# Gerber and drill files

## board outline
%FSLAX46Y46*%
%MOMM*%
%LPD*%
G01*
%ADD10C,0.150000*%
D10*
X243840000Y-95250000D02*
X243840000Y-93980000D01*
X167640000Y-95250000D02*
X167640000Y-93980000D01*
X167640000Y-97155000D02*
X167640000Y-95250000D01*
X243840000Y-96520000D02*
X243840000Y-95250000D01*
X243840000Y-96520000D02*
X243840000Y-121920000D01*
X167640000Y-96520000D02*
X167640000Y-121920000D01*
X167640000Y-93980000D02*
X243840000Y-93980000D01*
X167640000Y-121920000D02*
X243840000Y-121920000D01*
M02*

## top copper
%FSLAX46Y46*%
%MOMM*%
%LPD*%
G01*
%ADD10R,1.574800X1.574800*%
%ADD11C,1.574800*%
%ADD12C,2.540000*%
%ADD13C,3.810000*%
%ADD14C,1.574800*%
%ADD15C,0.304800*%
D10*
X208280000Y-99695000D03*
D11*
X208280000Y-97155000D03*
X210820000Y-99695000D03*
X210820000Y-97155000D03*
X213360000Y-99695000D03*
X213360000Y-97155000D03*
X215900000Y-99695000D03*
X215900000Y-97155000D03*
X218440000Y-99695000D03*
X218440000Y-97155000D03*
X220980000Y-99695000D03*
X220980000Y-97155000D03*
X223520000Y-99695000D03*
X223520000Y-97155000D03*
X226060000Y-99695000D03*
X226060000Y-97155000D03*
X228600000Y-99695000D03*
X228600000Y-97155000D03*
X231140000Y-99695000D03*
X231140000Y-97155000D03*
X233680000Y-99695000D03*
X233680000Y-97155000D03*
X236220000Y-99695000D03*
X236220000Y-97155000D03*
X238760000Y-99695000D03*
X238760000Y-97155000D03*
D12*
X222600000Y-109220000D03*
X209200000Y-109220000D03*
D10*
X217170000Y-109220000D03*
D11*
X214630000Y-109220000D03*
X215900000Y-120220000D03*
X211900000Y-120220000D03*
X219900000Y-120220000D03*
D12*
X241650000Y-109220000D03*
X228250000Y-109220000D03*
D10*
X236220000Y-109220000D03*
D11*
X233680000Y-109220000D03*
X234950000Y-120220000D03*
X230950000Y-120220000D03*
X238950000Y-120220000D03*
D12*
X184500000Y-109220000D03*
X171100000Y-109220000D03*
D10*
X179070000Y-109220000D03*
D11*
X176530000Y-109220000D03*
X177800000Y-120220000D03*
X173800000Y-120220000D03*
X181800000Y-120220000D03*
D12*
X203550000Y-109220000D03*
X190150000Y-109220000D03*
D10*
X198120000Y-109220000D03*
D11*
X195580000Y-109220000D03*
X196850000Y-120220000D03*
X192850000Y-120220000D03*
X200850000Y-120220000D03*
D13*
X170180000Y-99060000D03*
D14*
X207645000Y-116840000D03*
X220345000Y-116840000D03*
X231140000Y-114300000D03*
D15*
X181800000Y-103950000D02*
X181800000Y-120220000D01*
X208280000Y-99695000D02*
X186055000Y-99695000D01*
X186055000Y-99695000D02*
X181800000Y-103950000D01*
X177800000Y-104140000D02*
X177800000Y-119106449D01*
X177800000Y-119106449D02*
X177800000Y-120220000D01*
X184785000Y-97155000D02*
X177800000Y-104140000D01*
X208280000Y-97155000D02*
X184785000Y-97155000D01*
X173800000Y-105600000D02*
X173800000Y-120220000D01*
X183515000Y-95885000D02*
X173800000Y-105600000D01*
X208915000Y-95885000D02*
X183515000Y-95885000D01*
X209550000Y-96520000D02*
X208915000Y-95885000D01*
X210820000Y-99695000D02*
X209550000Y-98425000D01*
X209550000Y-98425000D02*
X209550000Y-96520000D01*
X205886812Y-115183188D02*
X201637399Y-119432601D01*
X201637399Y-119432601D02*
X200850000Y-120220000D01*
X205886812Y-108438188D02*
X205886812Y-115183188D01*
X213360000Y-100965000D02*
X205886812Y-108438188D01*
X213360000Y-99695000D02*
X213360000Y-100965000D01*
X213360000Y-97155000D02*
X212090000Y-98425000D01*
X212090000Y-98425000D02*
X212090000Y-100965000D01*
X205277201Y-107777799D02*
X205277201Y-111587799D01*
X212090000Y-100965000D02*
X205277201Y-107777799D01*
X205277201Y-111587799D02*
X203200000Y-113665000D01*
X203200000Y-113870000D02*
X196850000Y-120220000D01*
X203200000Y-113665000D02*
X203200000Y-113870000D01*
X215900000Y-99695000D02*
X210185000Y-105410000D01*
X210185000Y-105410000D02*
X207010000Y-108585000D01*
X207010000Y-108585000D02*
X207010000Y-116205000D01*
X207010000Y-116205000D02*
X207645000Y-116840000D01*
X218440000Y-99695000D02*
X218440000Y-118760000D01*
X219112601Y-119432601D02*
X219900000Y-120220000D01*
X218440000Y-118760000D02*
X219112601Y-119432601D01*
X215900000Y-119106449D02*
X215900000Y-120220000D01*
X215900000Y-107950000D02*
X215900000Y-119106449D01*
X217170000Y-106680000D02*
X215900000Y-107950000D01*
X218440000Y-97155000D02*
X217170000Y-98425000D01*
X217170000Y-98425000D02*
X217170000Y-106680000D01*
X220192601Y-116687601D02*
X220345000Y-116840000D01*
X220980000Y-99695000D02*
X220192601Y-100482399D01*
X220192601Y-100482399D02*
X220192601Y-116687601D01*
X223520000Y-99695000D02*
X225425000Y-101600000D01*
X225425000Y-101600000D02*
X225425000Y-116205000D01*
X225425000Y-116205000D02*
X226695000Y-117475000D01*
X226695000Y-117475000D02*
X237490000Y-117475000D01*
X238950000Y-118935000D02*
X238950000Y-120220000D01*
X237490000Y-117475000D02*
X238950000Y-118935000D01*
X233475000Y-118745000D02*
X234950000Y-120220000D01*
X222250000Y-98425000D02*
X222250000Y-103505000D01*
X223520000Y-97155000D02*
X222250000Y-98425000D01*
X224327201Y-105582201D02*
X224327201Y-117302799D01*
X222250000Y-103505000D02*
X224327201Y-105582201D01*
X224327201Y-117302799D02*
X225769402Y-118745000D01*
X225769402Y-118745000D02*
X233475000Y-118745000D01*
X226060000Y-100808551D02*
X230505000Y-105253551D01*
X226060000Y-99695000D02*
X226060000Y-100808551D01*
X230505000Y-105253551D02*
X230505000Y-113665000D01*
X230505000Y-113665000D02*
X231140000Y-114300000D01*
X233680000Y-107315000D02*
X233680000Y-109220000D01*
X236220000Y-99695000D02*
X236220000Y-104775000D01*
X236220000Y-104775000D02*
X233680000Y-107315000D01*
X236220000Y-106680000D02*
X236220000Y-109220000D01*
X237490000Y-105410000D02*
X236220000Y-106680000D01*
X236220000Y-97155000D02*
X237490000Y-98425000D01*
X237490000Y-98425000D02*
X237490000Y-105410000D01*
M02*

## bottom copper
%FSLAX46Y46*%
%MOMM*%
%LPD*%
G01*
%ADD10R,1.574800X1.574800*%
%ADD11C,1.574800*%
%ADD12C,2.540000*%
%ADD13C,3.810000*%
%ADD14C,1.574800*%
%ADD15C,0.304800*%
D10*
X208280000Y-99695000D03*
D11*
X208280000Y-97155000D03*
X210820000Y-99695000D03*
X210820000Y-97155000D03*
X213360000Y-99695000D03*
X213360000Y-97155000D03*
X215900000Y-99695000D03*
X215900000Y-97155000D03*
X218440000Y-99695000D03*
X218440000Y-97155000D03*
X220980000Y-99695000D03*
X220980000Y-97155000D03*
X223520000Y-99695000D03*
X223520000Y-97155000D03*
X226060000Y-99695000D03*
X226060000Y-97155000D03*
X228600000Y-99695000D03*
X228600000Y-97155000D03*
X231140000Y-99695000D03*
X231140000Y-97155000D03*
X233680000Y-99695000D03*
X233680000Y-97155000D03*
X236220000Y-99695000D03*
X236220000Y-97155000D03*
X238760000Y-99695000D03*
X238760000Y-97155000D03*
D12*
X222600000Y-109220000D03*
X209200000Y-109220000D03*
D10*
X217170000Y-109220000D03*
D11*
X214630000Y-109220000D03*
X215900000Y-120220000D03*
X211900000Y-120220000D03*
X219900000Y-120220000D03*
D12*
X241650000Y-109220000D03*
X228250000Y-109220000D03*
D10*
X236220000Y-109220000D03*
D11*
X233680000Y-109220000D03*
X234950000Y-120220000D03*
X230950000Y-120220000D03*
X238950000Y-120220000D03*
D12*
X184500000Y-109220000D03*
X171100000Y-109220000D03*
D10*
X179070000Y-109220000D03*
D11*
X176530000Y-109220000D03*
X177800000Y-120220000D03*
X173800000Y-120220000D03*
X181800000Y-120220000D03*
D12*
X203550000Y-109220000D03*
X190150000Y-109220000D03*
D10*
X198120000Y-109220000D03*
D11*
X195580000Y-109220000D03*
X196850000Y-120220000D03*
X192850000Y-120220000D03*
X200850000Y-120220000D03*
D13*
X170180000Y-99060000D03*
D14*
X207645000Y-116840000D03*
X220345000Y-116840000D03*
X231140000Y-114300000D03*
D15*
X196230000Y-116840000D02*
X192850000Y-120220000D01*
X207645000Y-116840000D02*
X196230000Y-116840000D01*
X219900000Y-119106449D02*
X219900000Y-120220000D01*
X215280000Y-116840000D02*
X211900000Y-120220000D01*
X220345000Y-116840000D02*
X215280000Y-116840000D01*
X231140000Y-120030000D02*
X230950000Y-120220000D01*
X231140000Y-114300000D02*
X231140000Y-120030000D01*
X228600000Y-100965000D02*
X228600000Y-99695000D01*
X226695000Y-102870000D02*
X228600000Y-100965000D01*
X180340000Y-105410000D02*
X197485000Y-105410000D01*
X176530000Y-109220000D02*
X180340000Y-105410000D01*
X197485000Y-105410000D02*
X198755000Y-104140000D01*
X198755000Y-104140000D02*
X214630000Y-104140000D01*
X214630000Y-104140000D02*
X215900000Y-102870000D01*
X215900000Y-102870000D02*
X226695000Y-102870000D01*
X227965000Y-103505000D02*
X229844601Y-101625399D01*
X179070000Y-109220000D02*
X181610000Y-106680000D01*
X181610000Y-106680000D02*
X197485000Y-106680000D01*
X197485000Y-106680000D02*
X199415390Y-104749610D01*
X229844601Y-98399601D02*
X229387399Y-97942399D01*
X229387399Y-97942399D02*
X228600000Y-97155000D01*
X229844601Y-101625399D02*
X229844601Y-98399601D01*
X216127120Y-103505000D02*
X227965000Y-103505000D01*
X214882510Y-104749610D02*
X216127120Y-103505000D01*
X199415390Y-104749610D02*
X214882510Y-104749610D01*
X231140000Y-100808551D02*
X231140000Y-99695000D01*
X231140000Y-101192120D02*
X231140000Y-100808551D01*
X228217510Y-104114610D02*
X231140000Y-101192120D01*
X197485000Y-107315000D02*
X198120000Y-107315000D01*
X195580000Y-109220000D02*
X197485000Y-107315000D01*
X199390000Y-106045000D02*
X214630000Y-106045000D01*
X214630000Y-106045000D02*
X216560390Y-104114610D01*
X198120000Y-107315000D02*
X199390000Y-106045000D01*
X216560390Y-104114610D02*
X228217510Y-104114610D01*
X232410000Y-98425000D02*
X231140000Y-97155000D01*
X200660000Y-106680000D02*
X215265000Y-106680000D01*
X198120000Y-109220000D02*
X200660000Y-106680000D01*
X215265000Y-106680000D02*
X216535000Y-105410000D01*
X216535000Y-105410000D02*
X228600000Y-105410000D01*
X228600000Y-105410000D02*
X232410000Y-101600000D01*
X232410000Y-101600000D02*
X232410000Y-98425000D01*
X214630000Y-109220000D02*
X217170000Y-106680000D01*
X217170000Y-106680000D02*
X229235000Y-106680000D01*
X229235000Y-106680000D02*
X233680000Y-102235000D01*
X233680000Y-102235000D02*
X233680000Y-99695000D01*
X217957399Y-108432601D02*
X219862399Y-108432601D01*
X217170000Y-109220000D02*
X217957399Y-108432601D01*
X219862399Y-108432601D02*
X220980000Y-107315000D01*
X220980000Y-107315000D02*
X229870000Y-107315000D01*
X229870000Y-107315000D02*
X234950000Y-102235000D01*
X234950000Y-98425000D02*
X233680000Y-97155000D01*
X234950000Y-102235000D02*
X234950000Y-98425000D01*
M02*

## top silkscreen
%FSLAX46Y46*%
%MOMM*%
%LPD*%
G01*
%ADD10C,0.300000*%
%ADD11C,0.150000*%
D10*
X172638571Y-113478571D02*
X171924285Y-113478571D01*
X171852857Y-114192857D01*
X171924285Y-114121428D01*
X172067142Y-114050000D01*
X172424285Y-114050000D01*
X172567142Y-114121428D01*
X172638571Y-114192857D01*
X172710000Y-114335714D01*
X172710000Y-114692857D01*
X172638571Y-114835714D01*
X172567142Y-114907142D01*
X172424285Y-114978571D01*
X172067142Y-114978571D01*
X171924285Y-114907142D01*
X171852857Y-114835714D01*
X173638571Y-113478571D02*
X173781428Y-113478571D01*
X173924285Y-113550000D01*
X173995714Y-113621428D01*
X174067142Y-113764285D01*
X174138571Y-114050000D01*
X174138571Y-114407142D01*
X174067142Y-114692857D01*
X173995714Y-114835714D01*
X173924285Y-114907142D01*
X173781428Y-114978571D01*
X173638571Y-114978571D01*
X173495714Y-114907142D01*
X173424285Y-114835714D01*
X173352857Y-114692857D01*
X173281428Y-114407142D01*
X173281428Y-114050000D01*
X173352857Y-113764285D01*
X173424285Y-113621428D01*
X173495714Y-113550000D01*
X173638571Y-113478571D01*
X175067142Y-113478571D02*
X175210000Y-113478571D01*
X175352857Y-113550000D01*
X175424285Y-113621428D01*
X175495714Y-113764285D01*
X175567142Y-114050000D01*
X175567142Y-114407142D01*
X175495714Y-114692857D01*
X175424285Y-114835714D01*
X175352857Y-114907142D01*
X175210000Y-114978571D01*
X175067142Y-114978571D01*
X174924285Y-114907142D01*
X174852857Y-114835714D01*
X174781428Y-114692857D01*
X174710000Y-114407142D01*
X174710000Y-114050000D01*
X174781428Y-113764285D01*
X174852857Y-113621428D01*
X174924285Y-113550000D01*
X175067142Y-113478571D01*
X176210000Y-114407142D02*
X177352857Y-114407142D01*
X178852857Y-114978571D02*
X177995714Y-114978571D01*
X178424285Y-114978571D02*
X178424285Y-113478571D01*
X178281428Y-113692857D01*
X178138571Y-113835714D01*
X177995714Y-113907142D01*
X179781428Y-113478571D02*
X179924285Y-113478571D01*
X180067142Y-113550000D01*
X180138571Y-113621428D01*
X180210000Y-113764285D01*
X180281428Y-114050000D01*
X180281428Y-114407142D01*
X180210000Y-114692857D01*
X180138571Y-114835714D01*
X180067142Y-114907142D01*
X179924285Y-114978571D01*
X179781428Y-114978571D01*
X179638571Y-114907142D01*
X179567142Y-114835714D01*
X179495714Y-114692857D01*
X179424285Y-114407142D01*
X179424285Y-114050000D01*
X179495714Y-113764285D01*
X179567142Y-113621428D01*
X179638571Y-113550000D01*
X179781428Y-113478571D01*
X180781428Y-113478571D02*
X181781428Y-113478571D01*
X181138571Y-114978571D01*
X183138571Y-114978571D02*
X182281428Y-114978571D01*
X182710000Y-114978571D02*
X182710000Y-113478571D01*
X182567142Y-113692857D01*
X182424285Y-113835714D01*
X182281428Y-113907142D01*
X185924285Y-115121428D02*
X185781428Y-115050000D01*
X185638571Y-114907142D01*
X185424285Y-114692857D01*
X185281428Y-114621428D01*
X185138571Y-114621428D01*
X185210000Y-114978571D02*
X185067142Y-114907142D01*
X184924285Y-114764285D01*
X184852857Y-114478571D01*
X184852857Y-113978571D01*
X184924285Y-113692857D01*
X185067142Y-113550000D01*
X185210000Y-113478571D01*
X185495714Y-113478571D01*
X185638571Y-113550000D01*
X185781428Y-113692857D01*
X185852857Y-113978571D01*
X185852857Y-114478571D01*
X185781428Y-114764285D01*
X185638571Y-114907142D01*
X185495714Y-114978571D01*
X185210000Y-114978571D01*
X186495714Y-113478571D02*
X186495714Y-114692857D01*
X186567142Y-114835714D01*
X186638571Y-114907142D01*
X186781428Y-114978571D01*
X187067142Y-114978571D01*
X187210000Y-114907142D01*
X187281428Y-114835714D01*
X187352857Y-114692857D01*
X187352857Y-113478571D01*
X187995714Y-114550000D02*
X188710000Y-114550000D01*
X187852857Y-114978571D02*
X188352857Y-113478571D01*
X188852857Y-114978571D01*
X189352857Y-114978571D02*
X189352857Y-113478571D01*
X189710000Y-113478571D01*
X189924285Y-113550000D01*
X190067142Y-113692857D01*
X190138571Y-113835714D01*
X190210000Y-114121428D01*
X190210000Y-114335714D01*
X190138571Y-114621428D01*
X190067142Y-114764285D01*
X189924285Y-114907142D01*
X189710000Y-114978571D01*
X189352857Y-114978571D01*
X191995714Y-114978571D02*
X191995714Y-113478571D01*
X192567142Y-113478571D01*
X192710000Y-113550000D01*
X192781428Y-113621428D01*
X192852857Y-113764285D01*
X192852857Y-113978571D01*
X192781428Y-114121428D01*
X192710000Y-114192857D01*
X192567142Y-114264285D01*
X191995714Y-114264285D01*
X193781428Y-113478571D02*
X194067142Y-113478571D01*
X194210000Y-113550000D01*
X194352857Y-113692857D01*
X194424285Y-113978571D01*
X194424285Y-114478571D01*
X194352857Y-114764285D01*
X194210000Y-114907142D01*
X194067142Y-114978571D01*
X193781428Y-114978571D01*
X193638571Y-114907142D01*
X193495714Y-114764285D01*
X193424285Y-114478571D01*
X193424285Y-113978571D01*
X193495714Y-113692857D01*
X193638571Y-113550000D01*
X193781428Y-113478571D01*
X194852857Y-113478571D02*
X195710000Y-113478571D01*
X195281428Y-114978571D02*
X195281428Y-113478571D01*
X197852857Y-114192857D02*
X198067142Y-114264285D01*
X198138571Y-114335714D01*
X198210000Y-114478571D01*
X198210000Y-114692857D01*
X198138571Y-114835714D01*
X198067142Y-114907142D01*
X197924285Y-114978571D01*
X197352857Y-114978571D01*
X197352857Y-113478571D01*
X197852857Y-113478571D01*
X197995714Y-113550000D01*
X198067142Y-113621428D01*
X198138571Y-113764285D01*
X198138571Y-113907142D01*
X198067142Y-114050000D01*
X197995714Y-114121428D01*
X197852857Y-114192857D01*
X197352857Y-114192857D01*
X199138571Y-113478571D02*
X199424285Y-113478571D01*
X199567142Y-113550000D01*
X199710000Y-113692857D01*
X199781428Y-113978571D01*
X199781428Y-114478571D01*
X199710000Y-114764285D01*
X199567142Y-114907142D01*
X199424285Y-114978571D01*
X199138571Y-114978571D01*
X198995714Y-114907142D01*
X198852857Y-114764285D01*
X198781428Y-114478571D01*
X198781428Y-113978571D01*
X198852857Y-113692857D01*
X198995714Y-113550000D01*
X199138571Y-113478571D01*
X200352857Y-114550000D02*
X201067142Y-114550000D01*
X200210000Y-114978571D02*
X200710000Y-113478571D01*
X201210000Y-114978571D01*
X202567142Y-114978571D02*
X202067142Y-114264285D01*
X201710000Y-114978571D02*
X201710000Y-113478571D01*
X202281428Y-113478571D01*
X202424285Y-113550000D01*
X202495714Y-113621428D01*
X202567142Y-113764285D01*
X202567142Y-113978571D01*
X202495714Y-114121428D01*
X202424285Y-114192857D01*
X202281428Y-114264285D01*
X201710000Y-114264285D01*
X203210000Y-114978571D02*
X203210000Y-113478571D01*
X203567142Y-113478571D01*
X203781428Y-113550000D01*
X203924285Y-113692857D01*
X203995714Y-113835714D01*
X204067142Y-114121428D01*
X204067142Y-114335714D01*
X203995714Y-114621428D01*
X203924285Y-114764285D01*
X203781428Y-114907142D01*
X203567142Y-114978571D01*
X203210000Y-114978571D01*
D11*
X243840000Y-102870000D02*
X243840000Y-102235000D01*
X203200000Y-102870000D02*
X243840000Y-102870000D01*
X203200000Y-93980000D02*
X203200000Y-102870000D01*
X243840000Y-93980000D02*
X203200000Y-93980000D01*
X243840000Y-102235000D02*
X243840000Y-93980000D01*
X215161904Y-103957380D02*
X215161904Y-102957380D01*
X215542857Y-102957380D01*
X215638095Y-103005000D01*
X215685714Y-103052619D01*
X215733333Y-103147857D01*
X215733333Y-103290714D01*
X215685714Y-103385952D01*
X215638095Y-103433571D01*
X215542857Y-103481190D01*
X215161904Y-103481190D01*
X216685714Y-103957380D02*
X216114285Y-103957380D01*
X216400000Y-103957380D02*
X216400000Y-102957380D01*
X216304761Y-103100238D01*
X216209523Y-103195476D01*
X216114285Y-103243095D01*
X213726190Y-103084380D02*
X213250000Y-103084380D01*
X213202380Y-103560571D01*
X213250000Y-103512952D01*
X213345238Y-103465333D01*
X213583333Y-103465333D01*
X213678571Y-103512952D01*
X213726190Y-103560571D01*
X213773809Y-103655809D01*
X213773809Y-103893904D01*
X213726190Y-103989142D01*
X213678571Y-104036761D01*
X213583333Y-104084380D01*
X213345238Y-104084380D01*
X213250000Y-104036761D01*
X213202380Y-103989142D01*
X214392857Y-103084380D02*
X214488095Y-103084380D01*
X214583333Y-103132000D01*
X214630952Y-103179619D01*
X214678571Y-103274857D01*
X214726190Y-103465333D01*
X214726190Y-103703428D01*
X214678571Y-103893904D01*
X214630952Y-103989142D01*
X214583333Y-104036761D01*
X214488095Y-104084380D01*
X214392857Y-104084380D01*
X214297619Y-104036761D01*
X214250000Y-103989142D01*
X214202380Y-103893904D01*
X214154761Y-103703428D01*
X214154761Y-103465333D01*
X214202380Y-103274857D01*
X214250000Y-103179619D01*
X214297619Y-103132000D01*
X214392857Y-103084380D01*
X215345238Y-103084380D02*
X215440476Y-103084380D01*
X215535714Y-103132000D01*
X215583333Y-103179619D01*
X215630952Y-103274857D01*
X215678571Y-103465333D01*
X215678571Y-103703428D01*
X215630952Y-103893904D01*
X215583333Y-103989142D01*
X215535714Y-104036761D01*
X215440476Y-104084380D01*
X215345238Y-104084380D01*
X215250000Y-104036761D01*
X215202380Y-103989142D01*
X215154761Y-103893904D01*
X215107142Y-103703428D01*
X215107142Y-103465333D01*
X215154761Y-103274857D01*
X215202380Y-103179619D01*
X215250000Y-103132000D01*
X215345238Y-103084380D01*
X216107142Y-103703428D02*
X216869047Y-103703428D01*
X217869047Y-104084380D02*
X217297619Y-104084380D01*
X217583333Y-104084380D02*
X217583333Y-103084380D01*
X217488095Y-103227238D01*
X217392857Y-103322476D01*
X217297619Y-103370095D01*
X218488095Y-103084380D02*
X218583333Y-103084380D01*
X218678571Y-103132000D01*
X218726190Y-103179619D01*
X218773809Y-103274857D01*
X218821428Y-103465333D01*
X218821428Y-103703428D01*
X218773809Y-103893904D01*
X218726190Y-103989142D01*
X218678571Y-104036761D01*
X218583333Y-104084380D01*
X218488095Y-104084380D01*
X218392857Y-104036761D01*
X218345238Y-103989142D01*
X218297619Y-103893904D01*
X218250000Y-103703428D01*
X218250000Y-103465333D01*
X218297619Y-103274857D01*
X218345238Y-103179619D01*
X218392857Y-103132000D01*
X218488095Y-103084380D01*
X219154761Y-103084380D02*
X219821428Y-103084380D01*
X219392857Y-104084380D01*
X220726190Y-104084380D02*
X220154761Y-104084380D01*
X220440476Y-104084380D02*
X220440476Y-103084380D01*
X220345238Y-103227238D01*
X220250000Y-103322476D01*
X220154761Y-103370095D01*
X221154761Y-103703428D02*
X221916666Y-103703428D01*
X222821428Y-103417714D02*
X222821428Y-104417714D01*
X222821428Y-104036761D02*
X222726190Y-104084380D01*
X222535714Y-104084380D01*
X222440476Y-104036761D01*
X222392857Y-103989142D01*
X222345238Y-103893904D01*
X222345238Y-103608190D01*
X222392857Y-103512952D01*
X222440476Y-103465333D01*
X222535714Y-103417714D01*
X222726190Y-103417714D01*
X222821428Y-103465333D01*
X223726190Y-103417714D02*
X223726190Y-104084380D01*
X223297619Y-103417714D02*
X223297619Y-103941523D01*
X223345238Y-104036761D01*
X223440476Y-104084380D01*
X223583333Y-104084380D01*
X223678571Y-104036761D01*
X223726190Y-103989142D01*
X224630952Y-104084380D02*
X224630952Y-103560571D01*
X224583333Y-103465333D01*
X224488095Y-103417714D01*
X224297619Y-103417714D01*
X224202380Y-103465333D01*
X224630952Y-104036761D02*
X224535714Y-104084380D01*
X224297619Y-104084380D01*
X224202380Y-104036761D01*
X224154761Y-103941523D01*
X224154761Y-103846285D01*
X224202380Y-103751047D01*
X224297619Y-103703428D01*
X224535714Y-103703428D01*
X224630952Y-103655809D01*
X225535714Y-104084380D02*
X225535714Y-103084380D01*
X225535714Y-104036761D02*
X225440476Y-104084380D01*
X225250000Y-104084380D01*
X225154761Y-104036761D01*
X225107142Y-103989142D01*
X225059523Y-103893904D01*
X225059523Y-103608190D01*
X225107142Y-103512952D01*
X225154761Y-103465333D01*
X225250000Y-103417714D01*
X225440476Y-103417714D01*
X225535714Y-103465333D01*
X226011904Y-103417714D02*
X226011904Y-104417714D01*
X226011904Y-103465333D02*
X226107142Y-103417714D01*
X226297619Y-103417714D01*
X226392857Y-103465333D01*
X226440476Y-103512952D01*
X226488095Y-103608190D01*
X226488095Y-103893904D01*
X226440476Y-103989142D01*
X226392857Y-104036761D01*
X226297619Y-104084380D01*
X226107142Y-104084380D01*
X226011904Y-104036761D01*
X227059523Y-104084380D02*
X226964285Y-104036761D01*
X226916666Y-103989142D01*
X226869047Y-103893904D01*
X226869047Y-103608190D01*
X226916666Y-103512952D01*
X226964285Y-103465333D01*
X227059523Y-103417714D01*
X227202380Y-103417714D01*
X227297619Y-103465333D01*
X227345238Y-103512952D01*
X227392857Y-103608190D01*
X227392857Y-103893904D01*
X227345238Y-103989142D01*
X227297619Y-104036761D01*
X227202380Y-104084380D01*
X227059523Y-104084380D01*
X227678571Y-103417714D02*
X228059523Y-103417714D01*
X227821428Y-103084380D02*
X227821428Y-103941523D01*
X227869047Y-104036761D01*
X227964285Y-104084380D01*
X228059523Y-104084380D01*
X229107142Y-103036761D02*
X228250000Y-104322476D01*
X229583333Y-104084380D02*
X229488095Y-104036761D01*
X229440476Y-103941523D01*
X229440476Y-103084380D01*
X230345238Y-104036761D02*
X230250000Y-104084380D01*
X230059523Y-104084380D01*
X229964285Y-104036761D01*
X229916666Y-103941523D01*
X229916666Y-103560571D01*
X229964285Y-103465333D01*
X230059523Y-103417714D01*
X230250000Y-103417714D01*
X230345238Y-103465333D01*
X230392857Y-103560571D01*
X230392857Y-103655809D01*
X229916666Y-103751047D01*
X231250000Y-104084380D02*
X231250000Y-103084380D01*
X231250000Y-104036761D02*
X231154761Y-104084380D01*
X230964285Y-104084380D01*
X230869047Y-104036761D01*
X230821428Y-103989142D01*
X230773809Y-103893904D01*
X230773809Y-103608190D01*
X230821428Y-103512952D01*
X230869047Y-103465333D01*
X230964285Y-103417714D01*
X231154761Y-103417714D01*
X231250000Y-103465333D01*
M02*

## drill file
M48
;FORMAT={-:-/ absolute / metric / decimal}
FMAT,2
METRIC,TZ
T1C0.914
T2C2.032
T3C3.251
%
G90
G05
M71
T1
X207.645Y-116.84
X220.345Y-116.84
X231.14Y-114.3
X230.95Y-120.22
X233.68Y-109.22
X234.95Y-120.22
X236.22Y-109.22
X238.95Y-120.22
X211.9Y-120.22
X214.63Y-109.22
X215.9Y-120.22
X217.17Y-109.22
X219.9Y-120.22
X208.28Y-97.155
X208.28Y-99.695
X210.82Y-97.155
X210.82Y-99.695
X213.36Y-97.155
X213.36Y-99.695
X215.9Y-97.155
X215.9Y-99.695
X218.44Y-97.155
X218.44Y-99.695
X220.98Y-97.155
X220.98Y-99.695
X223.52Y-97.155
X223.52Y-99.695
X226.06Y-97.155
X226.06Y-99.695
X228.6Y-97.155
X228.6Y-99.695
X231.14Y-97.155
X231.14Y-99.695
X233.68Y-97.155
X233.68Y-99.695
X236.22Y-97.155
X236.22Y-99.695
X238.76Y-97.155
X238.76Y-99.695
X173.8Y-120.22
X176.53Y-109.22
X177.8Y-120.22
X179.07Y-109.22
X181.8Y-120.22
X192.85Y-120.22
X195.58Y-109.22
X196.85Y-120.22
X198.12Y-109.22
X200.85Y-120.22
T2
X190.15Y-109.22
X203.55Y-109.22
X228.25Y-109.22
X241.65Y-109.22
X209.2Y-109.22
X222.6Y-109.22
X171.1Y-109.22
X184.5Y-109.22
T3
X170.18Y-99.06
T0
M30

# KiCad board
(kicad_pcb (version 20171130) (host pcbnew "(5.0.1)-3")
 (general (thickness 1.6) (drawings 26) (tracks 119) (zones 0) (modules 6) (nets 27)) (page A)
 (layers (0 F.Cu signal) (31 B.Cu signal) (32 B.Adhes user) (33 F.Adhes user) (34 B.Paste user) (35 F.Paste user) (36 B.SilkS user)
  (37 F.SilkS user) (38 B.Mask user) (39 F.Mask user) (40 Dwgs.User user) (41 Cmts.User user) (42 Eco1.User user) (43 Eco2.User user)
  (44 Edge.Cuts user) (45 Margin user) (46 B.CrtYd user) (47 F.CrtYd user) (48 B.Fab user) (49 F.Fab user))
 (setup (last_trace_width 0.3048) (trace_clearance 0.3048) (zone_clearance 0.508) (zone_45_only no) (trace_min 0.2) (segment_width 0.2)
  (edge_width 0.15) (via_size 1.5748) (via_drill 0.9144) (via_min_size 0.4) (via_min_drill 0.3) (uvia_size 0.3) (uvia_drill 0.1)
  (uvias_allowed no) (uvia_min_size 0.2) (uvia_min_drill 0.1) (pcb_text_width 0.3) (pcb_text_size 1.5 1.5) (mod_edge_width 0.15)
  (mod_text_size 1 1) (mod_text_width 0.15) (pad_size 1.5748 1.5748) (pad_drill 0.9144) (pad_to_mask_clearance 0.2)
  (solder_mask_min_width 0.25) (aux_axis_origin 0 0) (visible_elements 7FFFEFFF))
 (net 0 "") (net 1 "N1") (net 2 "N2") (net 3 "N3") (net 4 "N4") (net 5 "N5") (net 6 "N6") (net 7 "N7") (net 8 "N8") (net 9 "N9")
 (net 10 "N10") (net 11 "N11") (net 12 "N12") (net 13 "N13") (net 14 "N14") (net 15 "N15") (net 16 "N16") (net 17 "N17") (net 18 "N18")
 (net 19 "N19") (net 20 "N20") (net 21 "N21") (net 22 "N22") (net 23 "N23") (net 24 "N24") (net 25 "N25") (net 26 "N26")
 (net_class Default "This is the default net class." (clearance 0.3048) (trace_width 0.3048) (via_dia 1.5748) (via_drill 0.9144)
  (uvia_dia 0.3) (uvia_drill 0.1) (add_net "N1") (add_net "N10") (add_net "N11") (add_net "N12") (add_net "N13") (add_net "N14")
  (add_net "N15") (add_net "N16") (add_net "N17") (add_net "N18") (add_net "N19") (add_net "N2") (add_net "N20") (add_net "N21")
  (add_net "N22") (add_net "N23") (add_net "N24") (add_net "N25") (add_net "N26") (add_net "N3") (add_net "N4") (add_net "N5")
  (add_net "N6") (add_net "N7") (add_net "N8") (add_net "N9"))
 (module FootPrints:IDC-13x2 (layer F.Cu) (at 215.9 99.695)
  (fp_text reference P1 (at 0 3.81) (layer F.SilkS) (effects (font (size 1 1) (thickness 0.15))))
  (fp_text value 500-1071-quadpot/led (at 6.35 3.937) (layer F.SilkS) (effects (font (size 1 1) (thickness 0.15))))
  (fp_line (start 27.94 3.175) (end 27.94 2.54) (layer F.SilkS) (width 0.15))
  (fp_line (start -12.7 3.175) (end 27.94 3.175) (layer F.SilkS) (width 0.15))
  (fp_line (start -12.7 -5.715) (end -12.7 3.175) (layer F.SilkS) (width 0.15))
  (fp_line (start 27.94 -5.715) (end -12.7 -5.715) (layer F.SilkS) (width 0.15))
  (fp_line (start 27.94 2.54) (end 27.94 -5.715) (layer F.SilkS) (width 0.15))
  (pad 1 thru_hole rect (at -7.62 0) (size 1.5748 1.5748) (drill 0.9144) (layers *.Cu *.Mask) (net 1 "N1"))
  (pad 2 thru_hole circle (at -7.62 -2.54) (size 1.5748 1.5748) (drill 0.9144) (layers *.Cu *.Mask) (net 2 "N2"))
  (pad 3 thru_hole circle (at -5.08 0) (size 1.5748 1.5748) (drill 0.9144) (layers *.Cu *.Mask) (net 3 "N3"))
  (pad 4 thru_hole circle (at -5.08 -2.54) (size 1.5748 1.5748) (drill 0.9144) (layers *.Cu *.Mask) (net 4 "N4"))
  (pad 5 thru_hole circle (at -2.54 0) (size 1.5748 1.5748) (drill 0.9144) (layers *.Cu *.Mask) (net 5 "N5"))
  (pad 6 thru_hole circle (at -2.54 -2.54) (size 1.5748 1.5748) (drill 0.9144) (layers *.Cu *.Mask) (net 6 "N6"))
  (pad 7 thru_hole circle (at 0 0) (size 1.5748 1.5748) (drill 0.9144) (layers *.Cu *.Mask) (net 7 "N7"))
  (pad 8 thru_hole circle (at 0 -2.54) (size 1.5748 1.5748) (drill 0.9144) (layers *.Cu *.Mask) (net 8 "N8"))
  (pad 9 thru_hole circle (at 2.54 0) (size 1.5748 1.5748) (drill 0.9144) (layers *.Cu *.Mask) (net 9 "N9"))
  (pad 10 thru_hole circle (at 2.54 -2.54) (size 1.5748 1.5748) (drill 0.9144) (layers *.Cu *.Mask) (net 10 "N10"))
  (pad 11 thru_hole circle (at 5.08 0) (size 1.5748 1.5748) (drill 0.9144) (layers *.Cu *.Mask) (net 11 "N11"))
  (pad 12 thru_hole circle (at 5.08 -2.54) (size 1.5748 1.5748) (drill 0.9144) (layers *.Cu *.Mask) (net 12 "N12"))
  (pad 13 thru_hole circle (at 7.62 0) (size 1.5748 1.5748) (drill 0.9144) (layers *.Cu *.Mask) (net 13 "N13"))
  (pad 14 thru_hole circle (at 7.62 -2.54) (size 1.5748 1.5748) (drill 0.9144) (layers *.Cu *.Mask) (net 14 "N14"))
  (pad 15 thru_hole circle (at 10.16 0) (size 1.5748 1.5748) (drill 0.9144) (layers *.Cu *.Mask) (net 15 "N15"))
  (pad 16 thru_hole circle (at 10.16 -2.54) (size 1.5748 1.5748) (drill 0.9144) (layers *.Cu *.Mask) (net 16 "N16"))
  (pad 17 thru_hole circle (at 12.7 0) (size 1.5748 1.5748) (drill 0.9144) (layers *.Cu *.Mask) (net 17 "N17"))
  (pad 18 thru_hole circle (at 12.7 -2.54) (size 1.5748 1.5748) (drill 0.9144) (layers *.Cu *.Mask) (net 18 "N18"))
  (pad 19 thru_hole circle (at 15.24 0) (size 1.5748 1.5748) (drill 0.9144) (layers *.Cu *.Mask) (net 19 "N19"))
  (pad 20 thru_hole circle (at 15.24 -2.54) (size 1.5748 1.5748) (drill 0.9144) (layers *.Cu *.Mask) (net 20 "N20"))
  (pad 21 thru_hole circle (at 17.78 0) (size 1.5748 1.5748) (drill 0.9144) (layers *.Cu *.Mask) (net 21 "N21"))
  (pad 22 thru_hole circle (at 17.78 -2.54) (size 1.5748 1.5748) (drill 0.9144) (layers *.Cu *.Mask) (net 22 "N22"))
  (pad 23 thru_hole circle (at 20.32 0) (size 1.5748 1.5748) (drill 0.9144) (layers *.Cu *.Mask) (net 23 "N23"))
  (pad 24 thru_hole circle (at 20.32 -2.54) (size 1.5748 1.5748) (drill 0.9144) (layers *.Cu *.Mask) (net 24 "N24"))
  (pad 25 thru_hole circle (at 22.86 0) (size 1.5748 1.5748) (drill 0.9144) (layers *.Cu *.Mask) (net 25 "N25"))
  (pad 26 thru_hole circle (at 22.86 -2.54) (size 1.5748 1.5748) (drill 0.9144) (layers *.Cu *.Mask) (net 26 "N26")))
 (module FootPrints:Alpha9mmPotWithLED (layer B.Cu) (at 215.9 109.22 180)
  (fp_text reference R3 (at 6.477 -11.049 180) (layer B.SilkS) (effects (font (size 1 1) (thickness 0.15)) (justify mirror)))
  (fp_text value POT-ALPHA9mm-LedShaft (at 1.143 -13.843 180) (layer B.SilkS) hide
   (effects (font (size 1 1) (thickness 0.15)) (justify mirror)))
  (pad "" thru_hole circle (at -6.7 0 180) (size 2.54 2.54) (drill 2.032) (layers *.Cu *.Mask B.SilkS))
  (pad "" thru_hole circle (at 6.7 0 180) (size 2.54 2.54) (drill 2.032) (layers *.Cu *.Mask B.SilkS))
  (pad 4 thru_hole rect (at -1.27 0 180) (size 1.5748 1.5748) (drill 0.9144) (layers *.Cu *.Mask B.SilkS) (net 22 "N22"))
  (pad 5 thru_hole circle (at 1.27 0 180) (size 1.5748 1.5748) (drill 0.9144) (layers *.Cu *.Mask B.SilkS) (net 21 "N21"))
  (pad 2 thru_hole circle (at 0 -11 180) (size 1.5748 1.5748) (drill 0.9144) (layers *.Cu *.Mask B.SilkS) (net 10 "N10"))
  (pad 3 thru_hole circle (at 4 -11 180) (size 1.5748 1.5748) (drill 0.9144) (layers *.Cu *.Mask B.SilkS) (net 11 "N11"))
  (pad 1 thru_hole circle (at -4 -11 180) (size 1.5748 1.5748) (drill 0.9144) (layers *.Cu *.Mask B.SilkS) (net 9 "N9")))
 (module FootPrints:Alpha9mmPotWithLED (layer B.Cu) (at 234.95 109.22 180)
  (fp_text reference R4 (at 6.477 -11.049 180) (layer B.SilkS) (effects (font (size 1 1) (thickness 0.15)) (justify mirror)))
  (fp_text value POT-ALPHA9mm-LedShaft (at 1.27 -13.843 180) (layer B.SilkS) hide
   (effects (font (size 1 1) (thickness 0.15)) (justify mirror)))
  (pad "" thru_hole circle (at -6.7 0 180) (size 2.54 2.54) (drill 2.032) (layers *.Cu *.Mask B.SilkS))
  (pad "" thru_hole circle (at 6.7 0 180) (size 2.54 2.54) (drill 2.032) (layers *.Cu *.Mask B.SilkS))
  (pad 4 thru_hole rect (at -1.27 0 180) (size 1.5748 1.5748) (drill 0.9144) (layers *.Cu *.Mask B.SilkS) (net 24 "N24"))
  (pad 5 thru_hole circle (at 1.27 0 180) (size 1.5748 1.5748) (drill 0.9144) (layers *.Cu *.Mask B.SilkS) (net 23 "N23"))
  (pad 2 thru_hole circle (at 0 -11 180) (size 1.5748 1.5748) (drill 0.9144) (layers *.Cu *.Mask B.SilkS) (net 14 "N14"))
  (pad 3 thru_hole circle (at 4 -11 180) (size 1.5748 1.5748) (drill 0.9144) (layers *.Cu *.Mask B.SilkS) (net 15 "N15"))
  (pad 1 thru_hole circle (at -4 -11 180) (size 1.5748 1.5748) (drill 0.9144) (layers *.Cu *.Mask B.SilkS) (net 13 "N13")))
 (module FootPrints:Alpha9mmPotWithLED (layer B.Cu) (at 177.8 109.22 180)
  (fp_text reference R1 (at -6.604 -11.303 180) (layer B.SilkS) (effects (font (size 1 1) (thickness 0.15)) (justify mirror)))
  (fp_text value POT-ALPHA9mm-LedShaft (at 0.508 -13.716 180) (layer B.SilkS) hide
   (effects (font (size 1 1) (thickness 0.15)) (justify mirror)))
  (pad "" thru_hole circle (at -6.7 0 180) (size 2.54 2.54) (drill 2.032) (layers *.Cu *.Mask B.SilkS))
  (pad "" thru_hole circle (at 6.7 0 180) (size 2.54 2.54) (drill 2.032) (layers *.Cu *.Mask B.SilkS))
  (pad 4 thru_hole rect (at -1.27 0 180) (size 1.5748 1.5748) (drill 0.9144) (layers *.Cu *.Mask B.SilkS) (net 18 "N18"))
  (pad 5 thru_hole circle (at 1.27 0 180) (size 1.5748 1.5748) (drill 0.9144) (layers *.Cu *.Mask B.SilkS) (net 17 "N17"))
  (pad 2 thru_hole circle (at 0 -11 180) (size 1.5748 1.5748) (drill 0.9144) (layers *.Cu *.Mask B.SilkS) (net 2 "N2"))
  (pad 3 thru_hole circle (at 4 -11 180) (size 1.5748 1.5748) (drill 0.9144) (layers *.Cu *.Mask B.SilkS) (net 3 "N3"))
  (pad 1 thru_hole circle (at -4 -11 180) (size 1.5748 1.5748) (drill 0.9144) (layers *.Cu *.Mask B.SilkS) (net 1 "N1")))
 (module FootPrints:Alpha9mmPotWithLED (layer B.Cu) (at 196.85 109.22 180)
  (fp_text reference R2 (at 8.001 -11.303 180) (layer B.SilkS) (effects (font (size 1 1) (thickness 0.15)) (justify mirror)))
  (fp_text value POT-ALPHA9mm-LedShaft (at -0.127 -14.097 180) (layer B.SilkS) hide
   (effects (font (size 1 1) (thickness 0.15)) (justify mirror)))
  (pad "" thru_hole circle (at -6.7 0 180) (size 2.54 2.54) (drill 2.032) (layers *.Cu *.Mask B.SilkS))
  (pad "" thru_hole circle (at 6.7 0 180) (size 2.54 2.54) (drill 2.032) (layers *.Cu *.Mask B.SilkS))
  (pad 4 thru_hole rect (at -1.27 0 180) (size 1.5748 1.5748) (drill 0.9144) (layers *.Cu *.Mask B.SilkS) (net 20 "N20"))
  (pad 5 thru_hole circle (at 1.27 0 180) (size 1.5748 1.5748) (drill 0.9144) (layers *.Cu *.Mask B.SilkS) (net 19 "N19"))
  (pad 2 thru_hole circle (at 0 -11 180) (size 1.5748 1.5748) (drill 0.9144) (layers *.Cu *.Mask B.SilkS) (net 6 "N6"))
  (pad 3 thru_hole circle (at 4 -11 180) (size 1.5748 1.5748) (drill 0.9144) (layers *.Cu *.Mask B.SilkS) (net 7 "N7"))
  (pad 1 thru_hole circle (at -4 -11 180) (size 1.5748 1.5748) (drill 0.9144) (layers *.Cu *.Mask B.SilkS) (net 5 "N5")))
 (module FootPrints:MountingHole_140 (layer F.Cu) (at 170.18 99.06)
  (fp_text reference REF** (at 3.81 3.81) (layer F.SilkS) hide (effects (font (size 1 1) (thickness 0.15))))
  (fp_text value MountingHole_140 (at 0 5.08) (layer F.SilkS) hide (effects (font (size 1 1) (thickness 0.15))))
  (pad "" thru_hole circle (at 0 0) (size 3.81 3.81) (drill 3.2512) (layers *.Cu *.Mask F.SilkS)))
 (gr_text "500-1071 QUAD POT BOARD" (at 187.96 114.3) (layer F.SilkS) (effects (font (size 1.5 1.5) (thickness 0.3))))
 (gr_line (start 243.84 95.25) (end 243.84 93.98) (layer Edge.Cuts) (width 0.15))
 (gr_line (start 167.64 95.25) (end 167.64 93.98) (layer Edge.Cuts) (width 0.15))
 (gr_line (start 167.64 97.155) (end 167.64 95.25) (layer Edge.Cuts) (width 0.15))
 (gr_line (start 243.84 96.52) (end 243.84 95.25) (layer Edge.Cuts) (width 0.15))
 (gr_line (start 243.84 96.52) (end 243.84 121.92) (layer Edge.Cuts) (width 0.15))
 (gr_line (start 167.64 96.52) (end 167.64 121.92) (layer Edge.Cuts) (width 0.15))
 (gr_line (start 167.64 93.98) (end 243.84 93.98) (layer Edge.Cuts) (width 0.15))
 (gr_line (start 167.64 121.92) (end 243.84 121.92) (layer Edge.Cuts) (width 0.15))
 (segment (start 181.8 103.95) (end 181.8 120.22) (width 0.3048) (layer F.Cu) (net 1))
 (segment (start 208.28 99.695) (end 186.055 99.695) (width 0.3048) (layer F.Cu) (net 1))
 (segment (start 186.055 99.695) (end 181.8 103.95) (width 0.3048) (layer F.Cu) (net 1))
 (segment (start 177.8 104.14) (end 177.8 119.106449) (width 0.3048) (layer F.Cu) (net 2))
 (segment (start 177.8 119.106449) (end 177.8 120.22) (width 0.3048) (layer F.Cu) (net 2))
 (segment (start 184.785 97.155) (end 177.8 104.14) (width 0.3048) (layer F.Cu) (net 2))
 (segment (start 208.28 97.155) (end 184.785 97.155) (width 0.3048) (layer F.Cu) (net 2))
 (segment (start 173.8 105.6) (end 173.8 120.22) (width 0.3048) (layer F.Cu) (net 3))
 (segment (start 183.515 95.885) (end 173.8 105.6) (width 0.3048) (layer F.Cu) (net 3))
 (segment (start 208.915 95.885) (end 183.515 95.885) (width 0.3048) (layer F.Cu) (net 3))
 (segment (start 209.55 96.52) (end 208.915 95.885) (width 0.3048) (layer F.Cu) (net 3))
 (segment (start 210.82 99.695) (end 209.55 98.425) (width 0.3048) (layer F.Cu) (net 3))
 (segment (start 209.55 98.425) (end 209.55 96.52) (width 0.3048) (layer F.Cu) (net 3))
 (segment (start 205.886812 115.183188) (end 201.637399 119.432601) (width 0.3048) (layer F.Cu) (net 5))
 (segment (start 201.637399 119.432601) (end 200.85 120.22) (width 0.3048) (layer F.Cu) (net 5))
 (segment (start 205.886812 108.438188) (end 205.886812 115.183188) (width 0.3048) (layer F.Cu) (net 5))
 (segment (start 213.36 100.965) (end 205.886812 108.438188) (width 0.3048) (layer F.Cu) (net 5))
 (segment (start 213.36 99.695) (end 213.36 100.965) (width 0.3048) (layer F.Cu) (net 5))
 (segment (start 213.36 97.155) (end 212.09 98.425) (width 0.3048) (layer F.Cu) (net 6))
 (segment (start 212.09 98.425) (end 212.09 100.965) (width 0.3048) (layer F.Cu) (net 6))
 (segment (start 205.277201 107.777799) (end 205.277201 111.587799) (width 0.3048) (layer F.Cu) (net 6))
 (segment (start 212.09 100.965) (end 205.277201 107.777799) (width 0.3048) (layer F.Cu) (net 6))
 (segment (start 205.277201 111.587799) (end 203.2 113.665) (width 0.3048) (layer F.Cu) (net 6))
 (segment (start 203.2 113.87) (end 196.85 120.22) (width 0.3048) (layer F.Cu) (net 6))
 (segment (start 203.2 113.665) (end 203.2 113.87) (width 0.3048) (layer F.Cu) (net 6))
 (segment (start 215.9 99.695) (end 210.185 105.41) (width 0.3048) (layer F.Cu) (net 7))
 (segment (start 210.185 105.41) (end 207.01 108.585) (width 0.3048) (layer F.Cu) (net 7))
 (via (at 207.645 116.84) (size 1.5748) (drill 0.9144) (layers F.Cu B.Cu) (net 7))
 (segment (start 207.01 108.585) (end 207.01 116.205) (width 0.3048) (layer F.Cu) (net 7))
 (segment (start 207.01 116.205) (end 207.645 116.84) (width 0.3048) (layer F.Cu) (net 7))
 (segment (start 196.23 116.84) (end 192.85 120.22) (width 0.3048) (layer B.Cu) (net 7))
 (segment (start 207.645 116.84) (end 196.23 116.84) (width 0.3048) (layer B.Cu) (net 7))
 (segment (start 219.9 119.106449) (end 219.9 120.22) (width 0.3048) (layer B.Cu) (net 9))
 (segment (start 218.44 99.695) (end 218.44 118.76) (width 0.3048) (layer F.Cu) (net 9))
 (segment (start 219.112601 119.432601) (end 219.9 120.22) (width 0.3048) (layer F.Cu) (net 9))
 (segment (start 218.44 118.76) (end 219.112601 119.432601) (width 0.3048) (layer F.Cu) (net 9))
 (segment (start 215.9 119.106449) (end 215.9 120.22) (width 0.3048) (layer F.Cu) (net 10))
 (segment (start 215.9 107.95) (end 215.9 119.106449) (width 0.3048) (layer F.Cu) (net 10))
 (segment (start 217.17 106.68) (end 215.9 107.95) (width 0.3048) (layer F.Cu) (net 10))
 (segment (start 218.44 97.155) (end 217.17 98.425) (width 0.3048) (layer F.Cu) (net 10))
 (segment (start 217.17 98.425) (end 217.17 106.68) (width 0.3048) (layer F.Cu) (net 10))
 (via (at 220.345 116.84) (size 1.5748) (drill 0.9144) (layers F.Cu B.Cu) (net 11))
 (segment (start 220.192601 116.687601) (end 220.345 116.84) (width 0.3048) (layer F.Cu) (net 11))
 (segment (start 220.98 99.695) (end 220.192601 100.482399) (width 0.3048) (layer F.Cu) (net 11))
 (segment (start 220.192601 100.482399) (end 220.192601 116.687601) (width 0.3048) (layer F.Cu) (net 11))
 (segment (start 215.28 116.84) (end 211.9 120.22) (width 0.3048) (layer B.Cu) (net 11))
 (segment (start 220.345 116.84) (end 215.28 116.84) (width 0.3048) (layer B.Cu) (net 11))
 (segment (start 223.52 99.695) (end 225.425 101.6) (width 0.3048) (layer F.Cu) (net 13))
 (segment (start 225.425 101.6) (end 225.425 116.205) (width 0.3048) (layer F.Cu) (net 13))
 (segment (start 225.425 116.205) (end 226.695 117.475) (width 0.3048) (layer F.Cu) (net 13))
 (segment (start 226.695 117.475) (end 237.49 117.475) (width 0.3048) (layer F.Cu) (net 13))
 (segment (start 238.95 118.935) (end 238.95 120.22) (width 0.3048) (layer F.Cu) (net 13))
 (segment (start 237.49 117.475) (end 238.95 118.935) (width 0.3048) (layer F.Cu) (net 13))
 (segment (start 233.475 118.745) (end 234.95 120.22) (width 0.3048) (layer F.Cu) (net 14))
 (segment (start 222.25 98.425) (end 222.25 103.505) (width 0.3048) (layer F.Cu) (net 14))
 (segment (start 223.52 97.155) (end 222.25 98.425) (width 0.3048) (layer F.Cu) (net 14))
 (segment (start 224.327201 105.582201) (end 224.327201 117.302799) (width 0.3048) (layer F.Cu) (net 14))
 (segment (start 222.25 103.505) (end 224.327201 105.582201) (width 0.3048) (layer F.Cu) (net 14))
 (segment (start 224.327201 117.302799) (end 225.769402 118.745) (width 0.3048) (layer F.Cu) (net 14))
 (segment (start 225.769402 118.745) (end 233.475 118.745) (width 0.3048) (layer F.Cu) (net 14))
 (segment (start 226.06 100.808551) (end 230.505 105.253551) (width 0.3048) (layer F.Cu) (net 15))
 (segment (start 226.06 99.695) (end 226.06 100.808551) (width 0.3048) (layer F.Cu) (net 15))
 (segment (start 230.505 105.253551) (end 230.505 113.665) (width 0.3048) (layer F.Cu) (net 15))
 (via (at 231.14 114.3) (size 1.5748) (drill 0.9144) (layers F.Cu B.Cu) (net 15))
 (segment (start 230.505 113.665) (end 231.14 114.3) (width 0.3048) (layer F.Cu) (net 15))
 (segment (start 231.14 120.03) (end 230.95 120.22) (width 0.3048) (layer B.Cu) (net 15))
 (segment (start 231.14 114.3) (end 231.14 120.03) (width 0.3048) (layer B.Cu) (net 15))
 (segment (start 228.6 100.965) (end 228.6 99.695) (width 0.3048) (layer B.Cu) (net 17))
 (segment (start 226.695 102.87) (end 228.6 100.965) (width 0.3048) (layer B.Cu) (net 17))
 (segment (start 180.34 105.41) (end 197.485 105.41) (width 0.3048) (layer B.Cu) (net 17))
 (segment (start 176.53 109.22) (end 180.34 105.41) (width 0.3048) (layer B.Cu) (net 17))
 (segment (start 197.485 105.41) (end 198.755 104.14) (width 0.3048) (layer B.Cu) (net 17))
 (segment (start 198.755 104.14) (end 214.63 104.14) (width 0.3048) (layer B.Cu) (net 17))
 (segment (start 214.63 104.14) (end 215.9 102.87) (width 0.3048) (layer B.Cu) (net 17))
 (segment (start 215.9 102.87) (end 226.695 102.87) (width 0.3048) (layer B.Cu) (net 17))
 (segment (start 227.965 103.505) (end 229.844601 101.625399) (width 0.3048) (layer B.Cu) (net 18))
 (segment (start 179.07 109.22) (end 181.61 106.68) (width 0.3048) (layer B.Cu) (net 18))
 (segment (start 181.61 106.68) (end 197.485 106.68) (width 0.3048) (layer B.Cu) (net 18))
 (segment (start 197.485 106.68) (end 199.41539 104.74961) (width 0.3048) (layer B.Cu) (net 18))
 (segment (start 229.844601 98.399601) (end 229.387399 97.942399) (width 0.3048) (layer B.Cu) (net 18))
 (segment (start 229.387399 97.942399) (end 228.6 97.155) (width 0.3048) (layer B.Cu) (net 18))
 (segment (start 229.844601 101.625399) (end 229.844601 98.399601) (width 0.3048) (layer B.Cu) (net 18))
 (segment (start 216.12712 103.505) (end 227.965 103.505) (width 0.3048) (layer B.Cu) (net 18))
 (segment (start 214.88251 104.74961) (end 216.12712 103.505) (width 0.3048) (layer B.Cu) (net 18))
 (segment (start 199.41539 104.74961) (end 214.88251 104.74961) (width 0.3048) (layer B.Cu) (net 18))
 (segment (start 231.14 100.808551) (end 231.14 99.695) (width 0.3048) (layer B.Cu) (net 19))
 (segment (start 231.14 101.19212) (end 231.14 100.808551) (width 0.3048) (layer B.Cu) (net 19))
 (segment (start 228.21751 104.11461) (end 231.14 101.19212) (width 0.3048) (layer B.Cu) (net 19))
 (segment (start 197.485 107.315) (end 198.12 107.315) (width 0.3048) (layer B.Cu) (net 19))
 (segment (start 195.58 109.22) (end 197.485 107.315) (width 0.3048) (layer B.Cu) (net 19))
 (segment (start 199.39 106.045) (end 214.63 106.045) (width 0.3048) (layer B.Cu) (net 19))
 (segment (start 214.63 106.045) (end 216.56039 104.11461) (width 0.3048) (layer B.Cu) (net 19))
 (segment (start 198.12 107.315) (end 199.39 106.045) (width 0.3048) (layer B.Cu) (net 19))
 (segment (start 216.56039 104.11461) (end 228.21751 104.11461) (width 0.3048) (layer B.Cu) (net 19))
 (segment (start 232.41 98.425) (end 231.14 97.155) (width 0.3048) (layer B.Cu) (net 20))
 (segment (start 200.66 106.68) (end 215.265 106.68) (width 0.3048) (layer B.Cu) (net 20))
 (segment (start 198.12 109.22) (end 200.66 106.68) (width 0.3048) (layer B.Cu) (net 20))
 (segment (start 215.265 106.68) (end 216.535 105.41) (width 0.3048) (layer B.Cu) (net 20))
 (segment (start 216.535 105.41) (end 228.6 105.41) (width 0.3048) (layer B.Cu) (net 20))
 (segment (start 228.6 105.41) (end 232.41 101.6) (width 0.3048) (layer B.Cu) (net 20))
 (segment (start 232.41 101.6) (end 232.41 98.425) (width 0.3048) (layer B.Cu) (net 20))
 (segment (start 214.63 109.22) (end 217.17 106.68) (width 0.3048) (layer B.Cu) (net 21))
 (segment (start 217.17 106.68) (end 229.235 106.68) (width 0.3048) (layer B.Cu) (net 21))
 (segment (start 229.235 106.68) (end 233.68 102.235) (width 0.3048) (layer B.Cu) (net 21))
 (segment (start 233.68 102.235) (end 233.68 99.695) (width 0.3048) (layer B.Cu) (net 21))
 (segment (start 217.957399 108.432601) (end 219.862399 108.432601) (width 0.3048) (layer B.Cu) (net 22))
 (segment (start 217.17 109.22) (end 217.957399 108.432601) (width 0.3048) (layer B.Cu) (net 22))
 (segment (start 219.862399 108.432601) (end 220.98 107.315) (width 0.3048) (layer B.Cu) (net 22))
 (segment (start 220.98 107.315) (end 229.87 107.315) (width 0.3048) (layer B.Cu) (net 22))
 (segment (start 229.87 107.315) (end 234.95 102.235) (width 0.3048) (layer B.Cu) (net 22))
 (segment (start 234.95 98.425) (end 233.68 97.155) (width 0.3048) (layer B.Cu) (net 22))
 (segment (start 234.95 102.235) (end 234.95 98.425) (width 0.3048) (layer B.Cu) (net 22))
 (segment (start 233.68 107.315) (end 233.68 109.22) (width 0.3048) (layer F.Cu) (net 23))
 (segment (start 236.22 99.695) (end 236.22 104.775) (width 0.3048) (layer F.Cu) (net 23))
 (segment (start 236.22 104.775) (end 233.68 107.315) (width 0.3048) (layer F.Cu) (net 23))
 (segment (start 236.22 106.68) (end 236.22 109.22) (width 0.3048) (layer F.Cu) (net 24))
 (segment (start 237.49 105.41) (end 236.22 106.68) (width 0.3048) (layer F.Cu) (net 24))
 (segment (start 236.22 97.155) (end 237.49 98.425) (width 0.3048) (layer F.Cu) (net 24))
 (segment (start 237.49 98.425) (end 237.49 105.41) (width 0.3048) (layer F.Cu) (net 24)))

